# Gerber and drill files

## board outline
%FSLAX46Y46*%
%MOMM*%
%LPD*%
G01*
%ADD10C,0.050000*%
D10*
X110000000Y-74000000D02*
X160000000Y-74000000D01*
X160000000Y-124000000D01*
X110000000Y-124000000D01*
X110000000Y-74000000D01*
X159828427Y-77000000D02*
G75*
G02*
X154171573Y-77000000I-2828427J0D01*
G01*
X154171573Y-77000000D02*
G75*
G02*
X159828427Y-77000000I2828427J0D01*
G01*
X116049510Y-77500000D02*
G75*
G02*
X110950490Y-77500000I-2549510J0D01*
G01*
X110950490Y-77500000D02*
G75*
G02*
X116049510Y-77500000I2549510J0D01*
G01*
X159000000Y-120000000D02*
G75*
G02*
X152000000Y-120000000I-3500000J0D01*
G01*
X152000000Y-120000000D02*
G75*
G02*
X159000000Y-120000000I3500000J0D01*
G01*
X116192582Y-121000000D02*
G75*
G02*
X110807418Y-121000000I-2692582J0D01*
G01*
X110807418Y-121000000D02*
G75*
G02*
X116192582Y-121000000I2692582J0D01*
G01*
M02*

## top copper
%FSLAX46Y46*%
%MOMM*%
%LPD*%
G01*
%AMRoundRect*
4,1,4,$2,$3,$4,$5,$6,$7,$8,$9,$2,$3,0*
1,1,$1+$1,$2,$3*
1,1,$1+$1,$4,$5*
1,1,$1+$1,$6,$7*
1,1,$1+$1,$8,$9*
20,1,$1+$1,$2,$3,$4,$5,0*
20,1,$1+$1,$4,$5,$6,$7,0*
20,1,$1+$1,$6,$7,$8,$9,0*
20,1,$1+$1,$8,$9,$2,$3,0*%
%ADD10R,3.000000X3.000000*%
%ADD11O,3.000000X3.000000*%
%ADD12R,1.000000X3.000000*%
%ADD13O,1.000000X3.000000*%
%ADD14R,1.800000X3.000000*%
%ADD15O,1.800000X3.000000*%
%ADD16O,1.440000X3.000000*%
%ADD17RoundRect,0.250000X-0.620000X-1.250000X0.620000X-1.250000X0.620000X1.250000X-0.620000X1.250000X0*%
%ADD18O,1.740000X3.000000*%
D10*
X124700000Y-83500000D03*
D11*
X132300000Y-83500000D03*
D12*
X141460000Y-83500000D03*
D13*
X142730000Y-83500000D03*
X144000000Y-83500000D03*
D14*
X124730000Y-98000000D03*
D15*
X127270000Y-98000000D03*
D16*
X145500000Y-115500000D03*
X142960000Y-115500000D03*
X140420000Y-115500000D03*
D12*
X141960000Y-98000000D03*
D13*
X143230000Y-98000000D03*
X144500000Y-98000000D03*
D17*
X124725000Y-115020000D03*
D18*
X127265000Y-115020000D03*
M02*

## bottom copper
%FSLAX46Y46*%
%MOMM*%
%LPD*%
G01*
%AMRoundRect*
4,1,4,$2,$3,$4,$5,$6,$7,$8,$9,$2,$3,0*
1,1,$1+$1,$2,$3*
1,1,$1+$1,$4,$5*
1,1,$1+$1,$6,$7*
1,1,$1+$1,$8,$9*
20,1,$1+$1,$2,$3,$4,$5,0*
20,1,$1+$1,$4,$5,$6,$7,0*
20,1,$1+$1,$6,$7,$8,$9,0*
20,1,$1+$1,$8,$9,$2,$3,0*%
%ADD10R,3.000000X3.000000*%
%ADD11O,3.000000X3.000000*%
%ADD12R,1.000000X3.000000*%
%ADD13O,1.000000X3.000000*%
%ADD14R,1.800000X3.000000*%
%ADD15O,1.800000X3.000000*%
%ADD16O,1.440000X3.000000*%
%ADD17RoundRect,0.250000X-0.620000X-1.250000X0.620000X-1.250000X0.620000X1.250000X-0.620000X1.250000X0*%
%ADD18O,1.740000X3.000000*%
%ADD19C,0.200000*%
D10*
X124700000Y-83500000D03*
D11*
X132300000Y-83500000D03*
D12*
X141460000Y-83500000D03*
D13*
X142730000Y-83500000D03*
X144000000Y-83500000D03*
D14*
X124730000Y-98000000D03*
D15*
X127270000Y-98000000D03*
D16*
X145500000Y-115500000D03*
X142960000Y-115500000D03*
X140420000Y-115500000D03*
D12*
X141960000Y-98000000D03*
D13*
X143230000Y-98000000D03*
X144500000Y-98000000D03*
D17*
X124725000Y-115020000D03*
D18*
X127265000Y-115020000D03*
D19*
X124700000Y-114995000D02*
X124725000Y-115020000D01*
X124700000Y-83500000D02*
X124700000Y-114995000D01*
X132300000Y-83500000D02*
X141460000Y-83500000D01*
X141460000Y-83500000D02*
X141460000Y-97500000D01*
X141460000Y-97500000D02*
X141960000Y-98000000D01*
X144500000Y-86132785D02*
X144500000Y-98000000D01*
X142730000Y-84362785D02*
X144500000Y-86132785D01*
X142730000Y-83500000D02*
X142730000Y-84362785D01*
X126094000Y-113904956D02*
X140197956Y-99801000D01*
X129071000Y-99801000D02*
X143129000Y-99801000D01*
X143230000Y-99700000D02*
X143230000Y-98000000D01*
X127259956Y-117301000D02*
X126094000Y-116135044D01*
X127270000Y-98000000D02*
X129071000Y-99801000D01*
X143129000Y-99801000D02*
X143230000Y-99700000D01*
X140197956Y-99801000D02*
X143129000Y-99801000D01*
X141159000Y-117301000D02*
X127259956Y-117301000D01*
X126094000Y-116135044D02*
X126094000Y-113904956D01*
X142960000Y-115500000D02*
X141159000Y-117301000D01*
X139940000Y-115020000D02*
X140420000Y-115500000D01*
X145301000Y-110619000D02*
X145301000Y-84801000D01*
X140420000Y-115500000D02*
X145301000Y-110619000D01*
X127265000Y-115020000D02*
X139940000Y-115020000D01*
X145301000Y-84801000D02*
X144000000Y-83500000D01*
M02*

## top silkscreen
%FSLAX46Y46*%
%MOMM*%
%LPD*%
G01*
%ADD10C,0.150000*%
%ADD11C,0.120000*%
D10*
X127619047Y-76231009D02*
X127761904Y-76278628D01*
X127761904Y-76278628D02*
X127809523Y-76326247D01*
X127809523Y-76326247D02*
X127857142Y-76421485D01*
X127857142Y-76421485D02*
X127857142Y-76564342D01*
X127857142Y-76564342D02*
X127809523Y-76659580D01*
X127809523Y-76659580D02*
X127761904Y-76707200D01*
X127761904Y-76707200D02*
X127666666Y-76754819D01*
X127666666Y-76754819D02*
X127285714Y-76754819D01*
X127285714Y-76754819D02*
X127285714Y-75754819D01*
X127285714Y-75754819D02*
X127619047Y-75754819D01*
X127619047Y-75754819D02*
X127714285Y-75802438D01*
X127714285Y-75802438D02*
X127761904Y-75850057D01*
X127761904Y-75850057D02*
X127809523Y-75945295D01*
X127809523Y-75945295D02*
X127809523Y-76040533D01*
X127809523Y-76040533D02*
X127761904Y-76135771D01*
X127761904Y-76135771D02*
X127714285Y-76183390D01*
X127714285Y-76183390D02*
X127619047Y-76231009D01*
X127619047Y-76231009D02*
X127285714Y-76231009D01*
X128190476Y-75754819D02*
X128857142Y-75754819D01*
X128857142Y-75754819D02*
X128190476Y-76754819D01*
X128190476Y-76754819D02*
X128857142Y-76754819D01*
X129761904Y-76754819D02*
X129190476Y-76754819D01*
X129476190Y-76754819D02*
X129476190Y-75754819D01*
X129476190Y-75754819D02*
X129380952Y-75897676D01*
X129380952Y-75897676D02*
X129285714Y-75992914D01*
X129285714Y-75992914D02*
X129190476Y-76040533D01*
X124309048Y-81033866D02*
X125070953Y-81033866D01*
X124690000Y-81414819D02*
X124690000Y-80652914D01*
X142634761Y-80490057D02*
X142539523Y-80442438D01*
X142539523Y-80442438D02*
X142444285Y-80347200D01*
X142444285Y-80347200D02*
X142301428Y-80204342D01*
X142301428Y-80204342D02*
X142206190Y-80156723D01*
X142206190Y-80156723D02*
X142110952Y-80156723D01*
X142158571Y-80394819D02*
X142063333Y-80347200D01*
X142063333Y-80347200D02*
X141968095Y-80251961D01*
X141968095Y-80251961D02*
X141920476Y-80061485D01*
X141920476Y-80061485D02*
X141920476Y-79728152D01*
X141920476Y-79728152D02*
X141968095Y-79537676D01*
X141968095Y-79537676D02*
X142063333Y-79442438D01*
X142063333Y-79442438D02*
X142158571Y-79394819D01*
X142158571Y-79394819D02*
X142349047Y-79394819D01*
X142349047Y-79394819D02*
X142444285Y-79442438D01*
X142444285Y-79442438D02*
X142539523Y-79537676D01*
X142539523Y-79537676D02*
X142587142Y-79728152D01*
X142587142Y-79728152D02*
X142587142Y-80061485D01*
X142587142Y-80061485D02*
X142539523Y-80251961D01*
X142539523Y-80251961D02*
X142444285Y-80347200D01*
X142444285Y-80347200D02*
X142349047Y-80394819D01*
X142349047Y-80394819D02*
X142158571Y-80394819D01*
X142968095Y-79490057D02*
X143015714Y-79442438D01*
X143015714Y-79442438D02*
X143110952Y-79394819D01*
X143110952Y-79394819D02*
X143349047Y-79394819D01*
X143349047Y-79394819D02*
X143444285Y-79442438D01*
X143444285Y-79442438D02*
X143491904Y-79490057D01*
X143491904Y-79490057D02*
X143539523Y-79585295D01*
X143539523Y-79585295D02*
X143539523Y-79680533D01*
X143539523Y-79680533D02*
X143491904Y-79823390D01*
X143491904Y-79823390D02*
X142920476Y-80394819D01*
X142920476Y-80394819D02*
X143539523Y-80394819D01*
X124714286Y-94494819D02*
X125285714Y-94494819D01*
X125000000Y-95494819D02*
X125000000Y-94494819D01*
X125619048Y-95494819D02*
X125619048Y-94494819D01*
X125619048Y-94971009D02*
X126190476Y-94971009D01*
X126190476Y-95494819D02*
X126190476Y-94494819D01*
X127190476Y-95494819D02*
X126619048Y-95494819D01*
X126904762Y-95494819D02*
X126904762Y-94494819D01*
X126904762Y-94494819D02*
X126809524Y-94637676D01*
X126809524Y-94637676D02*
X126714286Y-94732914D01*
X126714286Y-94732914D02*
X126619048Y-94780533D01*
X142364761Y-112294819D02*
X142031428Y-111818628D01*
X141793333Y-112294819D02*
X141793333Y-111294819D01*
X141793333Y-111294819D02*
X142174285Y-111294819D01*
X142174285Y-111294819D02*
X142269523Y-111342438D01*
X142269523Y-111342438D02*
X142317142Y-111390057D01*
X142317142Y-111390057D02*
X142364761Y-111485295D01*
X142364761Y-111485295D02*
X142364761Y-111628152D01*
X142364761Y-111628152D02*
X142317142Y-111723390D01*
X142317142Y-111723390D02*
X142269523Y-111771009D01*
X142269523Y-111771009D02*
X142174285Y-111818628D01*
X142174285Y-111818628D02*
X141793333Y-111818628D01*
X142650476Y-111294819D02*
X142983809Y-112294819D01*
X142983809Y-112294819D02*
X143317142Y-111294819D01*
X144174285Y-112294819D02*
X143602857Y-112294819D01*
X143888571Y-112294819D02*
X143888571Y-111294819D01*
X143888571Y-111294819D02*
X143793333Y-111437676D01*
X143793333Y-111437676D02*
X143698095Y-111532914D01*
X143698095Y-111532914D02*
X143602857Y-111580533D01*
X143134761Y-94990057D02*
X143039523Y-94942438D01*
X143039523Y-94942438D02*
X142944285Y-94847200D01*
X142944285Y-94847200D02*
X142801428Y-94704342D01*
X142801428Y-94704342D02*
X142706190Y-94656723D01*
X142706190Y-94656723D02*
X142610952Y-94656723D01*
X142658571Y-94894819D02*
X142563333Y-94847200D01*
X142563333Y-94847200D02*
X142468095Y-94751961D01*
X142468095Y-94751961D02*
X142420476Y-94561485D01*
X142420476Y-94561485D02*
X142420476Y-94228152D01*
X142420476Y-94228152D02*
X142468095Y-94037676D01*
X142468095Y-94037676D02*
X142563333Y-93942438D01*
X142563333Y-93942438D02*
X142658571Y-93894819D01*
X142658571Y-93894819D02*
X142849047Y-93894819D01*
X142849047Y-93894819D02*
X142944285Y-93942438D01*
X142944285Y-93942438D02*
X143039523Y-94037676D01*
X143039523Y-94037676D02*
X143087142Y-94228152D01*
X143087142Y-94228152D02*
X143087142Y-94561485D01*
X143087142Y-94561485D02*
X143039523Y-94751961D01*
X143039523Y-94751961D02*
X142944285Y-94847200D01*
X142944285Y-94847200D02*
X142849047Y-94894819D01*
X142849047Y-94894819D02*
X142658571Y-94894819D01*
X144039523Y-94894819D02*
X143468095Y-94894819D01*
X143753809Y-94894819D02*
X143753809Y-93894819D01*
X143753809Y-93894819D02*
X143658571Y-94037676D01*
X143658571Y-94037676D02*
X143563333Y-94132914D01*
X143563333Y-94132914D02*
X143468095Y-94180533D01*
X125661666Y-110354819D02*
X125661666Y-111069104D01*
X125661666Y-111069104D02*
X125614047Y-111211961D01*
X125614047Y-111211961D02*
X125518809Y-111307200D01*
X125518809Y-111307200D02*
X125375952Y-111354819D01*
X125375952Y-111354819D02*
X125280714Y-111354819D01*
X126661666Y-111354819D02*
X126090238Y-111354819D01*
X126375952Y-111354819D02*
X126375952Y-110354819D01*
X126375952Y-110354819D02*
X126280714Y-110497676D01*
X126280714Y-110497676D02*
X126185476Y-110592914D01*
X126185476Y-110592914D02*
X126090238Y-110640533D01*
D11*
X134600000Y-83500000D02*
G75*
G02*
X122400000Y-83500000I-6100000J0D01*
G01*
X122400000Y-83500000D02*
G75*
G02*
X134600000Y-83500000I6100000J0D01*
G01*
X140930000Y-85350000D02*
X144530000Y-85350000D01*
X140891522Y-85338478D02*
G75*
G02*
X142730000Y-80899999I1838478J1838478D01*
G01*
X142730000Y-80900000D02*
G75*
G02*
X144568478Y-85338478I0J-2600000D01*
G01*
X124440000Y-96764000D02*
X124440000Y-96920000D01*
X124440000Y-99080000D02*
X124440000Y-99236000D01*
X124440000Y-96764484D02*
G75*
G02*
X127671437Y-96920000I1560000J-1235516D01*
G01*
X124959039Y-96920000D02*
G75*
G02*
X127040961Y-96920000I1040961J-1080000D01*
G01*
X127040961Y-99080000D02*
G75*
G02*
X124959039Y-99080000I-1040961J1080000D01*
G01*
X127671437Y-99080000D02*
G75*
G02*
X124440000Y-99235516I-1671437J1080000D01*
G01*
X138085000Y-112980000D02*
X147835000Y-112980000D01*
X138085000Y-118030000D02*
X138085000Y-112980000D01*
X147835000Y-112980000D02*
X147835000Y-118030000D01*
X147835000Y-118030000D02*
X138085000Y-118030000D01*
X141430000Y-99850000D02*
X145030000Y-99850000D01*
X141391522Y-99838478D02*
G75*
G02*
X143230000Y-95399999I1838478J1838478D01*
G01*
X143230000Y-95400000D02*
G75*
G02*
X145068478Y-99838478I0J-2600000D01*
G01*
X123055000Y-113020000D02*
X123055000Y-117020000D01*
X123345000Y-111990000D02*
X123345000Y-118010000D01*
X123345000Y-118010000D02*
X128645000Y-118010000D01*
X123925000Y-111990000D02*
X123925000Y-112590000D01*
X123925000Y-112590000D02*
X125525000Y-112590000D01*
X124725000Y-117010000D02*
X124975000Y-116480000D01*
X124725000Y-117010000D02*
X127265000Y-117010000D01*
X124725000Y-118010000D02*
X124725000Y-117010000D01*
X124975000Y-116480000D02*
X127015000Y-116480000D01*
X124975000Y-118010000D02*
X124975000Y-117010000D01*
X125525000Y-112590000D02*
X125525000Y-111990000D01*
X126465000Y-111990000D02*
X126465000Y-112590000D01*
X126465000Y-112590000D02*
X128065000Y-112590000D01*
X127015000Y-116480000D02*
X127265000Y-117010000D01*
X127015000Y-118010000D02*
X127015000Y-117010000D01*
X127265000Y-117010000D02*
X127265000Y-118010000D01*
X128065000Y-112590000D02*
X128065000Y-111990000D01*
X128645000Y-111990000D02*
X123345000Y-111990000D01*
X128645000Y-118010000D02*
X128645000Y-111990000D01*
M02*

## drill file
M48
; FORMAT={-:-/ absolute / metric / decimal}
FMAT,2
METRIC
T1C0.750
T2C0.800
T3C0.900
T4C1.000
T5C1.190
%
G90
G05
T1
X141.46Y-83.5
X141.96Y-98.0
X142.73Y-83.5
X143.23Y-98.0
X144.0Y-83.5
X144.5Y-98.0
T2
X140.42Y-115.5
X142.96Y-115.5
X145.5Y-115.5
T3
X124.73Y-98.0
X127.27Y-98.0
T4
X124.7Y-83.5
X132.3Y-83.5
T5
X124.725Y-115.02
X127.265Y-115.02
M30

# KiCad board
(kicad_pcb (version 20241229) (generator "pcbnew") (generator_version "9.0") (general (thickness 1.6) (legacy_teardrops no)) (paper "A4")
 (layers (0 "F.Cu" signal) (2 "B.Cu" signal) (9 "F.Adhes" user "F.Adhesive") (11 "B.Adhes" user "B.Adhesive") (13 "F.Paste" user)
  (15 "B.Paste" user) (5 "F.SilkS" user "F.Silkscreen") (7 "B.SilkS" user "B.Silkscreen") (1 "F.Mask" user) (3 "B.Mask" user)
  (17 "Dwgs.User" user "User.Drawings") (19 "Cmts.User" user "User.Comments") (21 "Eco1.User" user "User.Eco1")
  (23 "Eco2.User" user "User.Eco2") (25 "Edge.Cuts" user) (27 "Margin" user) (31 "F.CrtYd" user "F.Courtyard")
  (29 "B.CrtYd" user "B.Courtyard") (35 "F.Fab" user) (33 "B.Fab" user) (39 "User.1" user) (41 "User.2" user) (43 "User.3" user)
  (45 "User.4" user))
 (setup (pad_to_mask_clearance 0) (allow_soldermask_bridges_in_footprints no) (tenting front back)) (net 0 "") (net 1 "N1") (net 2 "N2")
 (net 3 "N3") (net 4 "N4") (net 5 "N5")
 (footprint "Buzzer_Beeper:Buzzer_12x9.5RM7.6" (layer "F.Cu") (at 124.7 83.5)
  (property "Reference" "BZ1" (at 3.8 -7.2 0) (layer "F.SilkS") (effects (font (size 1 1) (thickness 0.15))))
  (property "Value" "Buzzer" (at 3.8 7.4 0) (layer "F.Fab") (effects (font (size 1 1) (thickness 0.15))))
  (fp_circle (center 3.8 0) (end 9.9 0) (stroke (width 0.12) (type solid)) (fill no) (layer "F.SilkS"))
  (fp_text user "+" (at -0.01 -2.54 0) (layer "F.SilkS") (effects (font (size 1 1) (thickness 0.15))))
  (pad "1" thru_hole rect (at 0 0) (size 3 3) (drill 1) (layers "*.Cu" "*.Mask") (remove_unused_layers no) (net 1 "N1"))
  (pad "2" thru_hole oval (at 7.6 0) (size 3 3) (drill 1) (layers "*.Cu" "*.Mask") (remove_unused_layers no) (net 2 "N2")))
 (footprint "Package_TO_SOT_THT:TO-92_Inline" (layer "F.Cu") (at 141.46 83.5)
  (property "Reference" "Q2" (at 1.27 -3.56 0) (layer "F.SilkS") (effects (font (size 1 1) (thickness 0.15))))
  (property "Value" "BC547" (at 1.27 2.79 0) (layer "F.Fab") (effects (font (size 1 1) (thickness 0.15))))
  (fp_line (start -0.53 1.85) (end 3.07 1.85) (stroke (width 0.12) (type solid)) (layer "F.SilkS"))
  (fp_arc (start -0.568478 1.838478) (mid -1.132087 -0.994977) (end 1.27 -2.6) (stroke (width 0.12) (type solid)) (layer "F.SilkS"))
  (fp_arc (start 1.27 -2.6) (mid 3.672087 -0.994977) (end 3.108478 1.838478) (stroke (width 0.12) (type solid)) (layer "F.SilkS"))
  (pad "1" thru_hole rect (at 0 0) (size 1 3) (drill 0.75) (layers "*.Cu" "*.Mask") (remove_unused_layers no) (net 2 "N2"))
  (pad "2" thru_hole oval (at 1.27 0) (size 1 3) (drill 0.75) (layers "*.Cu" "*.Mask") (remove_unused_layers no) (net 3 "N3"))
  (pad "3" thru_hole oval (at 2.54 0) (size 1 3) (drill 0.75) (layers "*.Cu" "*.Mask") (remove_unused_layers no) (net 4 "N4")))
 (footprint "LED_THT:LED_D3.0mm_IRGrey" (layer "F.Cu") (at 124.73 98)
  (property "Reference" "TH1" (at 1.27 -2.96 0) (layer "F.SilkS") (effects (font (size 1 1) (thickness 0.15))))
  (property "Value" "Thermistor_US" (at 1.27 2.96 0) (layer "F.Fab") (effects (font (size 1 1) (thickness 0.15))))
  (fp_line (start -0.29 -1.236) (end -0.29 -1.08) (stroke (width 0.12) (type solid)) (layer "F.SilkS"))
  (fp_line (start -0.29 1.08) (end -0.29 1.236) (stroke (width 0.12) (type solid)) (layer "F.SilkS"))
  (fp_arc (start -0.29 -1.235516) (mid 1.36566 -1.987699) (end 2.941437 -1.08) (stroke (width 0.12) (type solid)) (layer "F.SilkS"))
  (fp_arc (start 0.229039 -1.08) (mid 1.27 -1.5) (end 2.310961 -1.08) (stroke (width 0.12) (type solid)) (layer "F.SilkS"))
  (fp_arc (start 2.310961 1.08) (mid 1.27 1.5) (end 0.229039 1.08) (stroke (width 0.12) (type solid)) (layer "F.SilkS"))
  (fp_arc (start 2.941437 1.08) (mid 1.36566 1.987699) (end -0.29 1.235516) (stroke (width 0.12) (type solid)) (layer "F.SilkS"))
  (pad "1" thru_hole rect (at 0 0) (size 1.8 3) (drill 0.9) (layers "*.Cu" "*.Mask") (remove_unused_layers no) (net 1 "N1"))
  (pad "2" thru_hole oval (at 2.54 0) (size 1.8 3) (drill 0.9) (layers "*.Cu" "*.Mask") (remove_unused_layers no) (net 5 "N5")))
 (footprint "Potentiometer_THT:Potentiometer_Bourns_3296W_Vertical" (layer "F.Cu") (at 145.5 115.5)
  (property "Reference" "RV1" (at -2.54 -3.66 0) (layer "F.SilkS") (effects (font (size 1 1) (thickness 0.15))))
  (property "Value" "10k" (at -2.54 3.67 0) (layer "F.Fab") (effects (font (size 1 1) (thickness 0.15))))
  (fp_line (start -7.415 -2.52) (end 2.335 -2.52) (stroke (width 0.12) (type solid)) (layer "F.SilkS"))
  (fp_line (start -7.415 2.53) (end -7.415 -2.52) (stroke (width 0.12) (type solid)) (layer "F.SilkS"))
  (fp_line (start 2.335 -2.52) (end 2.335 2.53) (stroke (width 0.12) (type solid)) (layer "F.SilkS"))
  (fp_line (start 2.335 2.53) (end -7.415 2.53) (stroke (width 0.12) (type solid)) (layer "F.SilkS"))
  (pad "1" thru_hole oval (at 0 0) (size 1.44 3) (drill 0.8) (layers "*.Cu" "*.Mask") (remove_unused_layers no) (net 5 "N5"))
  (pad "2" thru_hole oval (at -2.54 0) (size 1.44 3) (drill 0.8) (layers "*.Cu" "*.Mask") (remove_unused_layers no) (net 5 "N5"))
  (pad "3" thru_hole oval (at -5.08 0) (size 1.44 3) (drill 0.8) (layers "*.Cu" "*.Mask") (remove_unused_layers no) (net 4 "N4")))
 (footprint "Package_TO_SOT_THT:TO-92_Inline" (layer "F.Cu") (at 141.96 98)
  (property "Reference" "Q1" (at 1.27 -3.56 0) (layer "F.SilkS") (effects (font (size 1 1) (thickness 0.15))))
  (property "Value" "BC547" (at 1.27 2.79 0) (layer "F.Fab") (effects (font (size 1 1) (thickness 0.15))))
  (fp_line (start -0.53 1.85) (end 3.07 1.85) (stroke (width 0.12) (type solid)) (layer "F.SilkS"))
  (fp_arc (start -0.568478 1.838478) (mid -1.132087 -0.994977) (end 1.27 -2.6) (stroke (width 0.12) (type solid)) (layer "F.SilkS"))
  (fp_arc (start 1.27 -2.6) (mid 3.672087 -0.994977) (end 3.108478 1.838478) (stroke (width 0.12) (type solid)) (layer "F.SilkS"))
  (pad "1" thru_hole rect (at 0 0) (size 1 3) (drill 0.75) (layers "*.Cu" "*.Mask") (remove_unused_layers no) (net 2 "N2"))
  (pad "2" thru_hole oval (at 1.27 0) (size 1 3) (drill 0.75) (layers "*.Cu" "*.Mask") (remove_unused_layers no) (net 5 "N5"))
  (pad "3" thru_hole oval (at 2.54 0) (size 1 3) (drill 0.75) (layers "*.Cu" "*.Mask") (remove_unused_layers no) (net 3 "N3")))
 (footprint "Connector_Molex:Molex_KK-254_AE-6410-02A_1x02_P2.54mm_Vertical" (layer "F.Cu") (at 124.725 115.02)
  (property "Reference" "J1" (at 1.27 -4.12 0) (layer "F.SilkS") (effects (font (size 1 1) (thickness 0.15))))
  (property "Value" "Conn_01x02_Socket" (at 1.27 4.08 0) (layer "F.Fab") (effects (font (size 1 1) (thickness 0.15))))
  (fp_line (start -1.67 -2) (end -1.67 2) (stroke (width 0.12) (type solid)) (layer "F.SilkS"))
  (fp_line (start -1.38 -3.03) (end -1.38 2.99) (stroke (width 0.12) (type solid)) (layer "F.SilkS"))
  (fp_line (start -1.38 2.99) (end 3.92 2.99) (stroke (width 0.12) (type solid)) (layer "F.SilkS"))
  (fp_line (start -0.8 -3.03) (end -0.8 -2.43) (stroke (width 0.12) (type solid)) (layer "F.SilkS"))
  (fp_line (start -0.8 -2.43) (end 0.8 -2.43) (stroke (width 0.12) (type solid)) (layer "F.SilkS"))
  (fp_line (start 0 1.99) (end 0.25 1.46) (stroke (width 0.12) (type solid)) (layer "F.SilkS"))
  (fp_line (start 0 1.99) (end 2.54 1.99) (stroke (width 0.12) (type solid)) (layer "F.SilkS"))
  (fp_line (start 0 2.99) (end 0 1.99) (stroke (width 0.12) (type solid)) (layer "F.SilkS"))
  (fp_line (start 0.25 1.46) (end 2.29 1.46) (stroke (width 0.12) (type solid)) (layer "F.SilkS"))
  (fp_line (start 0.25 2.99) (end 0.25 1.99) (stroke (width 0.12) (type solid)) (layer "F.SilkS"))
  (fp_line (start 0.8 -2.43) (end 0.8 -3.03) (stroke (width 0.12) (type solid)) (layer "F.SilkS"))
  (fp_line (start 1.74 -3.03) (end 1.74 -2.43) (stroke (width 0.12) (type solid)) (layer "F.SilkS"))
  (fp_line (start 1.74 -2.43) (end 3.34 -2.43) (stroke (width 0.12) (type solid)) (layer "F.SilkS"))
  (fp_line (start 2.29 1.46) (end 2.54 1.99) (stroke (width 0.12) (type solid)) (layer "F.SilkS"))
  (fp_line (start 2.29 2.99) (end 2.29 1.99) (stroke (width 0.12) (type solid)) (layer "F.SilkS"))
  (fp_line (start 2.54 1.99) (end 2.54 2.99) (stroke (width 0.12) (type solid)) (layer "F.SilkS"))
  (fp_line (start 3.34 -2.43) (end 3.34 -3.03) (stroke (width 0.12) (type solid)) (layer "F.SilkS"))
  (fp_line (start 3.92 -3.03) (end -1.38 -3.03) (stroke (width 0.12) (type solid)) (layer "F.SilkS"))
  (fp_line (start 3.92 2.99) (end 3.92 -3.03) (stroke (width 0.12) (type solid)) (layer "F.SilkS"))
  (pad "1" thru_hole roundrect (at 0 0) (size 1.74 3) (drill 1.19) (layers "*.Cu" "*.Mask") (remove_unused_layers no)
   (roundrect_rratio 0.143678) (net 1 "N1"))
  (pad "2" thru_hole oval (at 2.54 0) (size 1.74 3) (drill 1.19) (layers "*.Cu" "*.Mask") (remove_unused_layers no) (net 4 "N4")))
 (gr_rect (start 110 74) (end 160 124) (stroke (width 0.05) (type default)) (fill no) (layer "Edge.Cuts"))
 (gr_circle (center 157 77) (end 159 79) (stroke (width 0.05) (type default)) (fill no) (layer "Edge.Cuts"))
 (gr_circle (center 113.5 77.5) (end 116 78) (stroke (width 0.05) (type default)) (fill no) (layer "Edge.Cuts"))
 (gr_circle (center 155.5 120) (end 159 120) (stroke (width 0.05) (type default)) (fill no) (layer "Edge.Cuts"))
 (gr_circle (center 113.5 121) (end 116 122) (stroke (width 0.05) (type default)) (fill no) (layer "Edge.Cuts"))
 (segment (start 124.7 114.995) (end 124.725 115.02) (width 0.2) (layer "B.Cu") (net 1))
 (segment (start 124.7 83.5) (end 124.7 114.995) (width 0.2) (layer "B.Cu") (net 1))
 (segment (start 132.3 83.5) (end 141.46 83.5) (width 0.2) (layer "B.Cu") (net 2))
 (segment (start 141.46 83.5) (end 141.46 97.5) (width 0.2) (layer "B.Cu") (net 2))
 (segment (start 141.46 97.5) (end 141.96 98) (width 0.2) (layer "B.Cu") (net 2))
 (segment (start 144.5 86.132785) (end 144.5 98) (width 0.2) (layer "B.Cu") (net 3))
 (segment (start 142.73 84.362785) (end 144.5 86.132785) (width 0.2) (layer "B.Cu") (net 3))
 (segment (start 142.73 83.5) (end 142.73 84.362785) (width 0.2) (layer "B.Cu") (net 3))
 (segment (start 126.094 113.904956) (end 140.197956 99.801) (width 0.2) (layer "B.Cu") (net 5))
 (segment (start 129.071 99.801) (end 143.129 99.801) (width 0.2) (layer "B.Cu") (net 5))
 (segment (start 143.23 99.7) (end 143.23 98) (width 0.2) (layer "B.Cu") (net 5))
 (segment (start 127.259956 117.301) (end 126.094 116.135044) (width 0.2) (layer "B.Cu") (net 5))
 (segment (start 127.27 98) (end 129.071 99.801) (width 0.2) (layer "B.Cu") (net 5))
 (segment (start 143.129 99.801) (end 143.23 99.7) (width 0.2) (layer "B.Cu") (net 5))
 (segment (start 140.197956 99.801) (end 143.129 99.801) (width 0.2) (layer "B.Cu") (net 5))
 (segment (start 141.159 117.301) (end 127.259956 117.301) (width 0.2) (layer "B.Cu") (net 5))
 (segment (start 126.094 116.135044) (end 126.094 113.904956) (width 0.2) (layer "B.Cu") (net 5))
 (segment (start 142.96 115.5) (end 141.159 117.301) (width 0.2) (layer "B.Cu") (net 5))
 (segment (start 139.94 115.02) (end 140.42 115.5) (width 0.2) (layer "B.Cu") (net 4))
 (segment (start 145.301 110.619) (end 145.301 84.801) (width 0.2) (layer "B.Cu") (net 4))
 (segment (start 140.42 115.5) (end 145.301 110.619) (width 0.2) (layer "B.Cu") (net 4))
 (segment (start 127.265 115.02) (end 139.94 115.02) (width 0.2) (layer "B.Cu") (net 4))
 (segment (start 145.301 84.801) (end 144 83.5) (width 0.2) (layer "B.Cu") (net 4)))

